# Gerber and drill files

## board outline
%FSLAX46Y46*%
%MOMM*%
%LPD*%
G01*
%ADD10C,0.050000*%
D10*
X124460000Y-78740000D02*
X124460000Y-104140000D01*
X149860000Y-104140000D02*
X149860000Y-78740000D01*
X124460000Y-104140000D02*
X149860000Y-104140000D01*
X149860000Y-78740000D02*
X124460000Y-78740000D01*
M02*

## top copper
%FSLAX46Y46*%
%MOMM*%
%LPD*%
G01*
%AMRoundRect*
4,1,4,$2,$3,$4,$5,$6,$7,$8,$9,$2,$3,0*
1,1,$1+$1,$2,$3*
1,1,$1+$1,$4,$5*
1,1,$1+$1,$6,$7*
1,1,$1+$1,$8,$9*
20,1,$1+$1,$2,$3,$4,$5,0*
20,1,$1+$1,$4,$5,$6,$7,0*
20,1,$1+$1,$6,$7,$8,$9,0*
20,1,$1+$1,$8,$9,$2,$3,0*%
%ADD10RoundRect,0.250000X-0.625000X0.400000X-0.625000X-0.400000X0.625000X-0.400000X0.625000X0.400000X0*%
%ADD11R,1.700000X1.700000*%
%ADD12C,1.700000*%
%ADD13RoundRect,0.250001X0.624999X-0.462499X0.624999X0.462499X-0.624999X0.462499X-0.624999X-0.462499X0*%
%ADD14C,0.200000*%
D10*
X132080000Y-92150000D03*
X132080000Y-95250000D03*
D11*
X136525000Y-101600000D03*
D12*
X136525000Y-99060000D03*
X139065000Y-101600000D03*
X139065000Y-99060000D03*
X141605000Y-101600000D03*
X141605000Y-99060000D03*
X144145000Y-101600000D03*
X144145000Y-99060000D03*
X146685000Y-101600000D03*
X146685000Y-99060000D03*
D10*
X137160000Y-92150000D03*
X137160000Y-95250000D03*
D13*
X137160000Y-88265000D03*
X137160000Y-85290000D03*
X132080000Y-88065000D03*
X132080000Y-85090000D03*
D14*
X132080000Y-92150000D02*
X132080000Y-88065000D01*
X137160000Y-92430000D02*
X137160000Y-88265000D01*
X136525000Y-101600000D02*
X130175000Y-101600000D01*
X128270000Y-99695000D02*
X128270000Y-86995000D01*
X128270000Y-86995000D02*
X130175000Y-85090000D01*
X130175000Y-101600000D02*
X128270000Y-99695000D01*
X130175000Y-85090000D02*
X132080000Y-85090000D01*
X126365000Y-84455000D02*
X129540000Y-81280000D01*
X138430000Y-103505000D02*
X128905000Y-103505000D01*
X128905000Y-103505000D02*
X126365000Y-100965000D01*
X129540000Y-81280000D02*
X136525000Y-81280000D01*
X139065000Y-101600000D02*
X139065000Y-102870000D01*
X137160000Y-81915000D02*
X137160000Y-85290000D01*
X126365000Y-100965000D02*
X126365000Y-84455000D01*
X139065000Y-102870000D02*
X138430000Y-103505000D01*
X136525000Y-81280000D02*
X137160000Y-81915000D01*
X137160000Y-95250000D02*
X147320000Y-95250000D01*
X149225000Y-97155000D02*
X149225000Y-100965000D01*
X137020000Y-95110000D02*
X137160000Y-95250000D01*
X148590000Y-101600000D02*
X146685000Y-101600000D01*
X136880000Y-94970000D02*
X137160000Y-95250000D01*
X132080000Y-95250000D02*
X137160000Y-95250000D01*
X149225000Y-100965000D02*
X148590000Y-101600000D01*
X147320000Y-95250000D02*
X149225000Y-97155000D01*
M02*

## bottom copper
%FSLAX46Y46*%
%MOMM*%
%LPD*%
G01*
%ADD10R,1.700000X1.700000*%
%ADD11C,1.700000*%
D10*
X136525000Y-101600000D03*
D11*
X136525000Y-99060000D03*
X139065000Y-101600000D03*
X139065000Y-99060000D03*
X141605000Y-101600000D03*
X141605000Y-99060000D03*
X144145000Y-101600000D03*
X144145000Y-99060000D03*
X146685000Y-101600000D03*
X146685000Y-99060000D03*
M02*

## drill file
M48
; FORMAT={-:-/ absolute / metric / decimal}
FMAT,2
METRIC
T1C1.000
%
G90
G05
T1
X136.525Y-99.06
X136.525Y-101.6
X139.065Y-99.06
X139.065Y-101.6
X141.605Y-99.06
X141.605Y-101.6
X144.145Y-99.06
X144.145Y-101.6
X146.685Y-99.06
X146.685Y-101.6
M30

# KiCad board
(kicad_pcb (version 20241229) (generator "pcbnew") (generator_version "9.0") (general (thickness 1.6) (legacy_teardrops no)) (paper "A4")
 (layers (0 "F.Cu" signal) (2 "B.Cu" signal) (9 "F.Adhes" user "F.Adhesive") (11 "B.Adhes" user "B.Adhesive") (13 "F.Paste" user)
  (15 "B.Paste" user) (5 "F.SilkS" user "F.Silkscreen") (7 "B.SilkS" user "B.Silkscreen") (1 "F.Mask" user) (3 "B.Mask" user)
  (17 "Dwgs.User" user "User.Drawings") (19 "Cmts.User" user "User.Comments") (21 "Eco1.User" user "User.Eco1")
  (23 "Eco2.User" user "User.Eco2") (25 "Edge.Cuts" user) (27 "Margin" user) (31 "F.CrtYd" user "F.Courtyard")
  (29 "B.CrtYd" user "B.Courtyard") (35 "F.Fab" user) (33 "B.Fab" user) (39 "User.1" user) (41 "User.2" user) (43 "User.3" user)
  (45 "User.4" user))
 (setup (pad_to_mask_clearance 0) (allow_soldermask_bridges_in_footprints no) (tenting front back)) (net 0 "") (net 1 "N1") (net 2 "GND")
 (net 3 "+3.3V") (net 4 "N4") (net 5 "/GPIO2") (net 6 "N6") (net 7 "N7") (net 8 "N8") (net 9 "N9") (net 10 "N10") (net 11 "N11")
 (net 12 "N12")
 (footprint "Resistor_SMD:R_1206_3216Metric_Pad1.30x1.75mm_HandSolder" (layer "F.Cu") (at 132.08 93.7 -90)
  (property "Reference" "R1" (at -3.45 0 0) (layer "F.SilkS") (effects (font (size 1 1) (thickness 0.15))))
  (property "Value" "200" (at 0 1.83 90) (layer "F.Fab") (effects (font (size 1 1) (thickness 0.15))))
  (pad "1" smd roundrect (at -1.55 0 270) (size 1.3 1.75) (layers "F.Cu" "F.Mask" "F.Paste") (roundrect_rratio 0.192308) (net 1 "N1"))
  (pad "2" smd roundrect (at 1.55 0 270) (size 1.3 1.75) (layers "F.Cu" "F.Mask" "F.Paste") (roundrect_rratio 0.192308) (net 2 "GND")))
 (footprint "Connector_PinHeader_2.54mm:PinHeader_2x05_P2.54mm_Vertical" (layer "F.Cu") (at 136.525 101.6 90)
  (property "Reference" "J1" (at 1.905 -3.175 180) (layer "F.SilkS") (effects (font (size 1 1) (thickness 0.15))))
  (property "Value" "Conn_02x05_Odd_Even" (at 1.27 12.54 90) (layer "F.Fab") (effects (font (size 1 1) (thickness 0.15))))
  (pad "1" thru_hole rect (at 0 0 90) (size 1.7 1.7) (drill 1) (layers "*.Cu" "*.Mask") (remove_unused_layers no) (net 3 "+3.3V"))
  (pad "2" thru_hole circle (at 2.54 0 90) (size 1.7 1.7) (drill 1) (layers "*.Cu" "*.Mask") (remove_unused_layers no) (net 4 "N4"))
  (pad "3" thru_hole circle (at 0 2.54 90) (size 1.7 1.7) (drill 1) (layers "*.Cu" "*.Mask") (remove_unused_layers no) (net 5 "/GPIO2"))
  (pad "4" thru_hole circle (at 2.54 2.54 90) (size 1.7 1.7) (drill 1) (layers "*.Cu" "*.Mask") (remove_unused_layers no) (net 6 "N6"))
  (pad "5" thru_hole circle (at 0 5.08 90) (size 1.7 1.7) (drill 1) (layers "*.Cu" "*.Mask") (remove_unused_layers no) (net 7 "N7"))
  (pad "6" thru_hole circle (at 2.54 5.08 90) (size 1.7 1.7) (drill 1) (layers "*.Cu" "*.Mask") (remove_unused_layers no) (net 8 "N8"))
  (pad "7" thru_hole circle (at 0 7.62 90) (size 1.7 1.7) (drill 1) (layers "*.Cu" "*.Mask") (remove_unused_layers no) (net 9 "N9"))
  (pad "8" thru_hole circle (at 2.54 7.62 90) (size 1.7 1.7) (drill 1) (layers "*.Cu" "*.Mask") (remove_unused_layers no) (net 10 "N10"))
  (pad "9" thru_hole circle (at 0 10.16 90) (size 1.7 1.7) (drill 1) (layers "*.Cu" "*.Mask") (remove_unused_layers no) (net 2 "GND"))
  (pad "10" thru_hole circle (at 2.54 10.16 90) (size 1.7 1.7) (drill 1) (layers "*.Cu" "*.Mask") (remove_unused_layers no) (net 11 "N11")))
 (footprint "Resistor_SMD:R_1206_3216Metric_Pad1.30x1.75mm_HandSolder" (layer "F.Cu") (at 137.16 93.7 -90)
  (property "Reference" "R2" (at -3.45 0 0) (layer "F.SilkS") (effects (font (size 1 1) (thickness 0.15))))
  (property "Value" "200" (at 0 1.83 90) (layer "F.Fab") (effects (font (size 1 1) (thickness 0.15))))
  (pad "1" smd roundrect (at -1.55 0 270) (size 1.3 1.75) (layers "F.Cu" "F.Mask" "F.Paste") (roundrect_rratio 0.192308) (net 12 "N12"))
  (pad "2" smd roundrect (at 1.55 0 270) (size 1.3 1.75) (layers "F.Cu" "F.Mask" "F.Paste") (roundrect_rratio 0.192308) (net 2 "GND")))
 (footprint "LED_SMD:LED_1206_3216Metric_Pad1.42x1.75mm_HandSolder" (layer "F.Cu") (at 137.16 86.7775 90)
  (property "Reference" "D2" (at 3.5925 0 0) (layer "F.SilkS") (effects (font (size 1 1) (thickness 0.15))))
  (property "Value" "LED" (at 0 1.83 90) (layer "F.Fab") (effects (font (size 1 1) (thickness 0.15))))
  (pad "1" smd roundrect (at -1.4875 0 90) (size 1.425 1.75) (layers "F.Cu" "F.Mask" "F.Paste") (roundrect_rratio 0.175439) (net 12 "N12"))
  (pad "2" smd roundrect (at 1.4875 0 90) (size 1.425 1.75) (layers "F.Cu" "F.Mask" "F.Paste") (roundrect_rratio 0.175439) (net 5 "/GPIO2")))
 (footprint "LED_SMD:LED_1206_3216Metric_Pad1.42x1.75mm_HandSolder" (layer "F.Cu") (at 132.08 86.5775 90)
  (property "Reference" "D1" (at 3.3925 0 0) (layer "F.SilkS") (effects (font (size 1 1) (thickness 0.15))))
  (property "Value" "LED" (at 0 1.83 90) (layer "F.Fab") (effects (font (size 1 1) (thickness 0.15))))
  (pad "1" smd roundrect (at -1.4875 0 90) (size 1.425 1.75) (layers "F.Cu" "F.Mask" "F.Paste") (roundrect_rratio 0.175439) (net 1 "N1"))
  (pad "2" smd roundrect (at 1.4875 0 90) (size 1.425 1.75) (layers "F.Cu" "F.Mask" "F.Paste") (roundrect_rratio 0.175439) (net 3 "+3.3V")))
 (gr_line (start 124.46 78.74) (end 124.46 104.14) (stroke (width 0.05) (type default)) (layer "Edge.Cuts"))
 (gr_line (start 149.86 104.14) (end 149.86 78.74) (stroke (width 0.05) (type default)) (layer "Edge.Cuts"))
 (gr_line (start 124.46 104.14) (end 149.86 104.14) (stroke (width 0.05) (type default)) (layer "Edge.Cuts"))
 (gr_line (start 149.86 78.74) (end 124.46 78.74) (stroke (width 0.05) (type default)) (layer "Edge.Cuts"))
 (segment (start 132.08 92.15) (end 132.08 88.065) (width 0.2) (layer "F.Cu") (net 1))
 (segment (start 137.16 92.43) (end 137.16 88.265) (width 0.2) (layer "F.Cu") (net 12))
 (segment (start 136.525 101.6) (end 130.175 101.6) (width 0.2) (layer "F.Cu") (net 3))
 (segment (start 128.27 99.695) (end 128.27 86.995) (width 0.2) (layer "F.Cu") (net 3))
 (segment (start 128.27 86.995) (end 130.175 85.09) (width 0.2) (layer "F.Cu") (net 3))
 (segment (start 130.175 101.6) (end 128.27 99.695) (width 0.2) (layer "F.Cu") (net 3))
 (segment (start 130.175 85.09) (end 132.08 85.09) (width 0.2) (layer "F.Cu") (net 3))
 (segment (start 126.365 84.455) (end 129.54 81.28) (width 0.2) (layer "F.Cu") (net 5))
 (segment (start 138.43 103.505) (end 128.905 103.505) (width 0.2) (layer "F.Cu") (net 5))
 (segment (start 128.905 103.505) (end 126.365 100.965) (width 0.2) (layer "F.Cu") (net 5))
 (segment (start 129.54 81.28) (end 136.525 81.28) (width 0.2) (layer "F.Cu") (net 5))
 (segment (start 139.065 101.6) (end 139.065 102.87) (width 0.2) (layer "F.Cu") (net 5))
 (segment (start 137.16 81.915) (end 137.16 85.29) (width 0.2) (layer "F.Cu") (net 5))
 (segment (start 126.365 100.965) (end 126.365 84.455) (width 0.2) (layer "F.Cu") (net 5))
 (segment (start 139.065 102.87) (end 138.43 103.505) (width 0.2) (layer "F.Cu") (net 5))
 (segment (start 136.525 81.28) (end 137.16 81.915) (width 0.2) (layer "F.Cu") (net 5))
 (segment (start 137.16 95.25) (end 147.32 95.25) (width 0.2) (layer "F.Cu") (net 2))
 (segment (start 149.225 97.155) (end 149.225 100.965) (width 0.2) (layer "F.Cu") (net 2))
 (segment (start 137.02 95.11) (end 137.16 95.25) (width 0.2) (layer "F.Cu") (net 2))
 (segment (start 148.59 101.6) (end 146.685 101.6) (width 0.2) (layer "F.Cu") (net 2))
 (segment (start 136.88 94.97) (end 137.16 95.25) (width 0.2) (layer "F.Cu") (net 2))
 (segment (start 132.08 95.25) (end 137.16 95.25) (width 0.2) (layer "F.Cu") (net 2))
 (segment (start 149.225 100.965) (end 148.59 101.6) (width 0.2) (layer "F.Cu") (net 2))
 (segment (start 147.32 95.25) (end 149.225 97.155) (width 0.2) (layer "F.Cu") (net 2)))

